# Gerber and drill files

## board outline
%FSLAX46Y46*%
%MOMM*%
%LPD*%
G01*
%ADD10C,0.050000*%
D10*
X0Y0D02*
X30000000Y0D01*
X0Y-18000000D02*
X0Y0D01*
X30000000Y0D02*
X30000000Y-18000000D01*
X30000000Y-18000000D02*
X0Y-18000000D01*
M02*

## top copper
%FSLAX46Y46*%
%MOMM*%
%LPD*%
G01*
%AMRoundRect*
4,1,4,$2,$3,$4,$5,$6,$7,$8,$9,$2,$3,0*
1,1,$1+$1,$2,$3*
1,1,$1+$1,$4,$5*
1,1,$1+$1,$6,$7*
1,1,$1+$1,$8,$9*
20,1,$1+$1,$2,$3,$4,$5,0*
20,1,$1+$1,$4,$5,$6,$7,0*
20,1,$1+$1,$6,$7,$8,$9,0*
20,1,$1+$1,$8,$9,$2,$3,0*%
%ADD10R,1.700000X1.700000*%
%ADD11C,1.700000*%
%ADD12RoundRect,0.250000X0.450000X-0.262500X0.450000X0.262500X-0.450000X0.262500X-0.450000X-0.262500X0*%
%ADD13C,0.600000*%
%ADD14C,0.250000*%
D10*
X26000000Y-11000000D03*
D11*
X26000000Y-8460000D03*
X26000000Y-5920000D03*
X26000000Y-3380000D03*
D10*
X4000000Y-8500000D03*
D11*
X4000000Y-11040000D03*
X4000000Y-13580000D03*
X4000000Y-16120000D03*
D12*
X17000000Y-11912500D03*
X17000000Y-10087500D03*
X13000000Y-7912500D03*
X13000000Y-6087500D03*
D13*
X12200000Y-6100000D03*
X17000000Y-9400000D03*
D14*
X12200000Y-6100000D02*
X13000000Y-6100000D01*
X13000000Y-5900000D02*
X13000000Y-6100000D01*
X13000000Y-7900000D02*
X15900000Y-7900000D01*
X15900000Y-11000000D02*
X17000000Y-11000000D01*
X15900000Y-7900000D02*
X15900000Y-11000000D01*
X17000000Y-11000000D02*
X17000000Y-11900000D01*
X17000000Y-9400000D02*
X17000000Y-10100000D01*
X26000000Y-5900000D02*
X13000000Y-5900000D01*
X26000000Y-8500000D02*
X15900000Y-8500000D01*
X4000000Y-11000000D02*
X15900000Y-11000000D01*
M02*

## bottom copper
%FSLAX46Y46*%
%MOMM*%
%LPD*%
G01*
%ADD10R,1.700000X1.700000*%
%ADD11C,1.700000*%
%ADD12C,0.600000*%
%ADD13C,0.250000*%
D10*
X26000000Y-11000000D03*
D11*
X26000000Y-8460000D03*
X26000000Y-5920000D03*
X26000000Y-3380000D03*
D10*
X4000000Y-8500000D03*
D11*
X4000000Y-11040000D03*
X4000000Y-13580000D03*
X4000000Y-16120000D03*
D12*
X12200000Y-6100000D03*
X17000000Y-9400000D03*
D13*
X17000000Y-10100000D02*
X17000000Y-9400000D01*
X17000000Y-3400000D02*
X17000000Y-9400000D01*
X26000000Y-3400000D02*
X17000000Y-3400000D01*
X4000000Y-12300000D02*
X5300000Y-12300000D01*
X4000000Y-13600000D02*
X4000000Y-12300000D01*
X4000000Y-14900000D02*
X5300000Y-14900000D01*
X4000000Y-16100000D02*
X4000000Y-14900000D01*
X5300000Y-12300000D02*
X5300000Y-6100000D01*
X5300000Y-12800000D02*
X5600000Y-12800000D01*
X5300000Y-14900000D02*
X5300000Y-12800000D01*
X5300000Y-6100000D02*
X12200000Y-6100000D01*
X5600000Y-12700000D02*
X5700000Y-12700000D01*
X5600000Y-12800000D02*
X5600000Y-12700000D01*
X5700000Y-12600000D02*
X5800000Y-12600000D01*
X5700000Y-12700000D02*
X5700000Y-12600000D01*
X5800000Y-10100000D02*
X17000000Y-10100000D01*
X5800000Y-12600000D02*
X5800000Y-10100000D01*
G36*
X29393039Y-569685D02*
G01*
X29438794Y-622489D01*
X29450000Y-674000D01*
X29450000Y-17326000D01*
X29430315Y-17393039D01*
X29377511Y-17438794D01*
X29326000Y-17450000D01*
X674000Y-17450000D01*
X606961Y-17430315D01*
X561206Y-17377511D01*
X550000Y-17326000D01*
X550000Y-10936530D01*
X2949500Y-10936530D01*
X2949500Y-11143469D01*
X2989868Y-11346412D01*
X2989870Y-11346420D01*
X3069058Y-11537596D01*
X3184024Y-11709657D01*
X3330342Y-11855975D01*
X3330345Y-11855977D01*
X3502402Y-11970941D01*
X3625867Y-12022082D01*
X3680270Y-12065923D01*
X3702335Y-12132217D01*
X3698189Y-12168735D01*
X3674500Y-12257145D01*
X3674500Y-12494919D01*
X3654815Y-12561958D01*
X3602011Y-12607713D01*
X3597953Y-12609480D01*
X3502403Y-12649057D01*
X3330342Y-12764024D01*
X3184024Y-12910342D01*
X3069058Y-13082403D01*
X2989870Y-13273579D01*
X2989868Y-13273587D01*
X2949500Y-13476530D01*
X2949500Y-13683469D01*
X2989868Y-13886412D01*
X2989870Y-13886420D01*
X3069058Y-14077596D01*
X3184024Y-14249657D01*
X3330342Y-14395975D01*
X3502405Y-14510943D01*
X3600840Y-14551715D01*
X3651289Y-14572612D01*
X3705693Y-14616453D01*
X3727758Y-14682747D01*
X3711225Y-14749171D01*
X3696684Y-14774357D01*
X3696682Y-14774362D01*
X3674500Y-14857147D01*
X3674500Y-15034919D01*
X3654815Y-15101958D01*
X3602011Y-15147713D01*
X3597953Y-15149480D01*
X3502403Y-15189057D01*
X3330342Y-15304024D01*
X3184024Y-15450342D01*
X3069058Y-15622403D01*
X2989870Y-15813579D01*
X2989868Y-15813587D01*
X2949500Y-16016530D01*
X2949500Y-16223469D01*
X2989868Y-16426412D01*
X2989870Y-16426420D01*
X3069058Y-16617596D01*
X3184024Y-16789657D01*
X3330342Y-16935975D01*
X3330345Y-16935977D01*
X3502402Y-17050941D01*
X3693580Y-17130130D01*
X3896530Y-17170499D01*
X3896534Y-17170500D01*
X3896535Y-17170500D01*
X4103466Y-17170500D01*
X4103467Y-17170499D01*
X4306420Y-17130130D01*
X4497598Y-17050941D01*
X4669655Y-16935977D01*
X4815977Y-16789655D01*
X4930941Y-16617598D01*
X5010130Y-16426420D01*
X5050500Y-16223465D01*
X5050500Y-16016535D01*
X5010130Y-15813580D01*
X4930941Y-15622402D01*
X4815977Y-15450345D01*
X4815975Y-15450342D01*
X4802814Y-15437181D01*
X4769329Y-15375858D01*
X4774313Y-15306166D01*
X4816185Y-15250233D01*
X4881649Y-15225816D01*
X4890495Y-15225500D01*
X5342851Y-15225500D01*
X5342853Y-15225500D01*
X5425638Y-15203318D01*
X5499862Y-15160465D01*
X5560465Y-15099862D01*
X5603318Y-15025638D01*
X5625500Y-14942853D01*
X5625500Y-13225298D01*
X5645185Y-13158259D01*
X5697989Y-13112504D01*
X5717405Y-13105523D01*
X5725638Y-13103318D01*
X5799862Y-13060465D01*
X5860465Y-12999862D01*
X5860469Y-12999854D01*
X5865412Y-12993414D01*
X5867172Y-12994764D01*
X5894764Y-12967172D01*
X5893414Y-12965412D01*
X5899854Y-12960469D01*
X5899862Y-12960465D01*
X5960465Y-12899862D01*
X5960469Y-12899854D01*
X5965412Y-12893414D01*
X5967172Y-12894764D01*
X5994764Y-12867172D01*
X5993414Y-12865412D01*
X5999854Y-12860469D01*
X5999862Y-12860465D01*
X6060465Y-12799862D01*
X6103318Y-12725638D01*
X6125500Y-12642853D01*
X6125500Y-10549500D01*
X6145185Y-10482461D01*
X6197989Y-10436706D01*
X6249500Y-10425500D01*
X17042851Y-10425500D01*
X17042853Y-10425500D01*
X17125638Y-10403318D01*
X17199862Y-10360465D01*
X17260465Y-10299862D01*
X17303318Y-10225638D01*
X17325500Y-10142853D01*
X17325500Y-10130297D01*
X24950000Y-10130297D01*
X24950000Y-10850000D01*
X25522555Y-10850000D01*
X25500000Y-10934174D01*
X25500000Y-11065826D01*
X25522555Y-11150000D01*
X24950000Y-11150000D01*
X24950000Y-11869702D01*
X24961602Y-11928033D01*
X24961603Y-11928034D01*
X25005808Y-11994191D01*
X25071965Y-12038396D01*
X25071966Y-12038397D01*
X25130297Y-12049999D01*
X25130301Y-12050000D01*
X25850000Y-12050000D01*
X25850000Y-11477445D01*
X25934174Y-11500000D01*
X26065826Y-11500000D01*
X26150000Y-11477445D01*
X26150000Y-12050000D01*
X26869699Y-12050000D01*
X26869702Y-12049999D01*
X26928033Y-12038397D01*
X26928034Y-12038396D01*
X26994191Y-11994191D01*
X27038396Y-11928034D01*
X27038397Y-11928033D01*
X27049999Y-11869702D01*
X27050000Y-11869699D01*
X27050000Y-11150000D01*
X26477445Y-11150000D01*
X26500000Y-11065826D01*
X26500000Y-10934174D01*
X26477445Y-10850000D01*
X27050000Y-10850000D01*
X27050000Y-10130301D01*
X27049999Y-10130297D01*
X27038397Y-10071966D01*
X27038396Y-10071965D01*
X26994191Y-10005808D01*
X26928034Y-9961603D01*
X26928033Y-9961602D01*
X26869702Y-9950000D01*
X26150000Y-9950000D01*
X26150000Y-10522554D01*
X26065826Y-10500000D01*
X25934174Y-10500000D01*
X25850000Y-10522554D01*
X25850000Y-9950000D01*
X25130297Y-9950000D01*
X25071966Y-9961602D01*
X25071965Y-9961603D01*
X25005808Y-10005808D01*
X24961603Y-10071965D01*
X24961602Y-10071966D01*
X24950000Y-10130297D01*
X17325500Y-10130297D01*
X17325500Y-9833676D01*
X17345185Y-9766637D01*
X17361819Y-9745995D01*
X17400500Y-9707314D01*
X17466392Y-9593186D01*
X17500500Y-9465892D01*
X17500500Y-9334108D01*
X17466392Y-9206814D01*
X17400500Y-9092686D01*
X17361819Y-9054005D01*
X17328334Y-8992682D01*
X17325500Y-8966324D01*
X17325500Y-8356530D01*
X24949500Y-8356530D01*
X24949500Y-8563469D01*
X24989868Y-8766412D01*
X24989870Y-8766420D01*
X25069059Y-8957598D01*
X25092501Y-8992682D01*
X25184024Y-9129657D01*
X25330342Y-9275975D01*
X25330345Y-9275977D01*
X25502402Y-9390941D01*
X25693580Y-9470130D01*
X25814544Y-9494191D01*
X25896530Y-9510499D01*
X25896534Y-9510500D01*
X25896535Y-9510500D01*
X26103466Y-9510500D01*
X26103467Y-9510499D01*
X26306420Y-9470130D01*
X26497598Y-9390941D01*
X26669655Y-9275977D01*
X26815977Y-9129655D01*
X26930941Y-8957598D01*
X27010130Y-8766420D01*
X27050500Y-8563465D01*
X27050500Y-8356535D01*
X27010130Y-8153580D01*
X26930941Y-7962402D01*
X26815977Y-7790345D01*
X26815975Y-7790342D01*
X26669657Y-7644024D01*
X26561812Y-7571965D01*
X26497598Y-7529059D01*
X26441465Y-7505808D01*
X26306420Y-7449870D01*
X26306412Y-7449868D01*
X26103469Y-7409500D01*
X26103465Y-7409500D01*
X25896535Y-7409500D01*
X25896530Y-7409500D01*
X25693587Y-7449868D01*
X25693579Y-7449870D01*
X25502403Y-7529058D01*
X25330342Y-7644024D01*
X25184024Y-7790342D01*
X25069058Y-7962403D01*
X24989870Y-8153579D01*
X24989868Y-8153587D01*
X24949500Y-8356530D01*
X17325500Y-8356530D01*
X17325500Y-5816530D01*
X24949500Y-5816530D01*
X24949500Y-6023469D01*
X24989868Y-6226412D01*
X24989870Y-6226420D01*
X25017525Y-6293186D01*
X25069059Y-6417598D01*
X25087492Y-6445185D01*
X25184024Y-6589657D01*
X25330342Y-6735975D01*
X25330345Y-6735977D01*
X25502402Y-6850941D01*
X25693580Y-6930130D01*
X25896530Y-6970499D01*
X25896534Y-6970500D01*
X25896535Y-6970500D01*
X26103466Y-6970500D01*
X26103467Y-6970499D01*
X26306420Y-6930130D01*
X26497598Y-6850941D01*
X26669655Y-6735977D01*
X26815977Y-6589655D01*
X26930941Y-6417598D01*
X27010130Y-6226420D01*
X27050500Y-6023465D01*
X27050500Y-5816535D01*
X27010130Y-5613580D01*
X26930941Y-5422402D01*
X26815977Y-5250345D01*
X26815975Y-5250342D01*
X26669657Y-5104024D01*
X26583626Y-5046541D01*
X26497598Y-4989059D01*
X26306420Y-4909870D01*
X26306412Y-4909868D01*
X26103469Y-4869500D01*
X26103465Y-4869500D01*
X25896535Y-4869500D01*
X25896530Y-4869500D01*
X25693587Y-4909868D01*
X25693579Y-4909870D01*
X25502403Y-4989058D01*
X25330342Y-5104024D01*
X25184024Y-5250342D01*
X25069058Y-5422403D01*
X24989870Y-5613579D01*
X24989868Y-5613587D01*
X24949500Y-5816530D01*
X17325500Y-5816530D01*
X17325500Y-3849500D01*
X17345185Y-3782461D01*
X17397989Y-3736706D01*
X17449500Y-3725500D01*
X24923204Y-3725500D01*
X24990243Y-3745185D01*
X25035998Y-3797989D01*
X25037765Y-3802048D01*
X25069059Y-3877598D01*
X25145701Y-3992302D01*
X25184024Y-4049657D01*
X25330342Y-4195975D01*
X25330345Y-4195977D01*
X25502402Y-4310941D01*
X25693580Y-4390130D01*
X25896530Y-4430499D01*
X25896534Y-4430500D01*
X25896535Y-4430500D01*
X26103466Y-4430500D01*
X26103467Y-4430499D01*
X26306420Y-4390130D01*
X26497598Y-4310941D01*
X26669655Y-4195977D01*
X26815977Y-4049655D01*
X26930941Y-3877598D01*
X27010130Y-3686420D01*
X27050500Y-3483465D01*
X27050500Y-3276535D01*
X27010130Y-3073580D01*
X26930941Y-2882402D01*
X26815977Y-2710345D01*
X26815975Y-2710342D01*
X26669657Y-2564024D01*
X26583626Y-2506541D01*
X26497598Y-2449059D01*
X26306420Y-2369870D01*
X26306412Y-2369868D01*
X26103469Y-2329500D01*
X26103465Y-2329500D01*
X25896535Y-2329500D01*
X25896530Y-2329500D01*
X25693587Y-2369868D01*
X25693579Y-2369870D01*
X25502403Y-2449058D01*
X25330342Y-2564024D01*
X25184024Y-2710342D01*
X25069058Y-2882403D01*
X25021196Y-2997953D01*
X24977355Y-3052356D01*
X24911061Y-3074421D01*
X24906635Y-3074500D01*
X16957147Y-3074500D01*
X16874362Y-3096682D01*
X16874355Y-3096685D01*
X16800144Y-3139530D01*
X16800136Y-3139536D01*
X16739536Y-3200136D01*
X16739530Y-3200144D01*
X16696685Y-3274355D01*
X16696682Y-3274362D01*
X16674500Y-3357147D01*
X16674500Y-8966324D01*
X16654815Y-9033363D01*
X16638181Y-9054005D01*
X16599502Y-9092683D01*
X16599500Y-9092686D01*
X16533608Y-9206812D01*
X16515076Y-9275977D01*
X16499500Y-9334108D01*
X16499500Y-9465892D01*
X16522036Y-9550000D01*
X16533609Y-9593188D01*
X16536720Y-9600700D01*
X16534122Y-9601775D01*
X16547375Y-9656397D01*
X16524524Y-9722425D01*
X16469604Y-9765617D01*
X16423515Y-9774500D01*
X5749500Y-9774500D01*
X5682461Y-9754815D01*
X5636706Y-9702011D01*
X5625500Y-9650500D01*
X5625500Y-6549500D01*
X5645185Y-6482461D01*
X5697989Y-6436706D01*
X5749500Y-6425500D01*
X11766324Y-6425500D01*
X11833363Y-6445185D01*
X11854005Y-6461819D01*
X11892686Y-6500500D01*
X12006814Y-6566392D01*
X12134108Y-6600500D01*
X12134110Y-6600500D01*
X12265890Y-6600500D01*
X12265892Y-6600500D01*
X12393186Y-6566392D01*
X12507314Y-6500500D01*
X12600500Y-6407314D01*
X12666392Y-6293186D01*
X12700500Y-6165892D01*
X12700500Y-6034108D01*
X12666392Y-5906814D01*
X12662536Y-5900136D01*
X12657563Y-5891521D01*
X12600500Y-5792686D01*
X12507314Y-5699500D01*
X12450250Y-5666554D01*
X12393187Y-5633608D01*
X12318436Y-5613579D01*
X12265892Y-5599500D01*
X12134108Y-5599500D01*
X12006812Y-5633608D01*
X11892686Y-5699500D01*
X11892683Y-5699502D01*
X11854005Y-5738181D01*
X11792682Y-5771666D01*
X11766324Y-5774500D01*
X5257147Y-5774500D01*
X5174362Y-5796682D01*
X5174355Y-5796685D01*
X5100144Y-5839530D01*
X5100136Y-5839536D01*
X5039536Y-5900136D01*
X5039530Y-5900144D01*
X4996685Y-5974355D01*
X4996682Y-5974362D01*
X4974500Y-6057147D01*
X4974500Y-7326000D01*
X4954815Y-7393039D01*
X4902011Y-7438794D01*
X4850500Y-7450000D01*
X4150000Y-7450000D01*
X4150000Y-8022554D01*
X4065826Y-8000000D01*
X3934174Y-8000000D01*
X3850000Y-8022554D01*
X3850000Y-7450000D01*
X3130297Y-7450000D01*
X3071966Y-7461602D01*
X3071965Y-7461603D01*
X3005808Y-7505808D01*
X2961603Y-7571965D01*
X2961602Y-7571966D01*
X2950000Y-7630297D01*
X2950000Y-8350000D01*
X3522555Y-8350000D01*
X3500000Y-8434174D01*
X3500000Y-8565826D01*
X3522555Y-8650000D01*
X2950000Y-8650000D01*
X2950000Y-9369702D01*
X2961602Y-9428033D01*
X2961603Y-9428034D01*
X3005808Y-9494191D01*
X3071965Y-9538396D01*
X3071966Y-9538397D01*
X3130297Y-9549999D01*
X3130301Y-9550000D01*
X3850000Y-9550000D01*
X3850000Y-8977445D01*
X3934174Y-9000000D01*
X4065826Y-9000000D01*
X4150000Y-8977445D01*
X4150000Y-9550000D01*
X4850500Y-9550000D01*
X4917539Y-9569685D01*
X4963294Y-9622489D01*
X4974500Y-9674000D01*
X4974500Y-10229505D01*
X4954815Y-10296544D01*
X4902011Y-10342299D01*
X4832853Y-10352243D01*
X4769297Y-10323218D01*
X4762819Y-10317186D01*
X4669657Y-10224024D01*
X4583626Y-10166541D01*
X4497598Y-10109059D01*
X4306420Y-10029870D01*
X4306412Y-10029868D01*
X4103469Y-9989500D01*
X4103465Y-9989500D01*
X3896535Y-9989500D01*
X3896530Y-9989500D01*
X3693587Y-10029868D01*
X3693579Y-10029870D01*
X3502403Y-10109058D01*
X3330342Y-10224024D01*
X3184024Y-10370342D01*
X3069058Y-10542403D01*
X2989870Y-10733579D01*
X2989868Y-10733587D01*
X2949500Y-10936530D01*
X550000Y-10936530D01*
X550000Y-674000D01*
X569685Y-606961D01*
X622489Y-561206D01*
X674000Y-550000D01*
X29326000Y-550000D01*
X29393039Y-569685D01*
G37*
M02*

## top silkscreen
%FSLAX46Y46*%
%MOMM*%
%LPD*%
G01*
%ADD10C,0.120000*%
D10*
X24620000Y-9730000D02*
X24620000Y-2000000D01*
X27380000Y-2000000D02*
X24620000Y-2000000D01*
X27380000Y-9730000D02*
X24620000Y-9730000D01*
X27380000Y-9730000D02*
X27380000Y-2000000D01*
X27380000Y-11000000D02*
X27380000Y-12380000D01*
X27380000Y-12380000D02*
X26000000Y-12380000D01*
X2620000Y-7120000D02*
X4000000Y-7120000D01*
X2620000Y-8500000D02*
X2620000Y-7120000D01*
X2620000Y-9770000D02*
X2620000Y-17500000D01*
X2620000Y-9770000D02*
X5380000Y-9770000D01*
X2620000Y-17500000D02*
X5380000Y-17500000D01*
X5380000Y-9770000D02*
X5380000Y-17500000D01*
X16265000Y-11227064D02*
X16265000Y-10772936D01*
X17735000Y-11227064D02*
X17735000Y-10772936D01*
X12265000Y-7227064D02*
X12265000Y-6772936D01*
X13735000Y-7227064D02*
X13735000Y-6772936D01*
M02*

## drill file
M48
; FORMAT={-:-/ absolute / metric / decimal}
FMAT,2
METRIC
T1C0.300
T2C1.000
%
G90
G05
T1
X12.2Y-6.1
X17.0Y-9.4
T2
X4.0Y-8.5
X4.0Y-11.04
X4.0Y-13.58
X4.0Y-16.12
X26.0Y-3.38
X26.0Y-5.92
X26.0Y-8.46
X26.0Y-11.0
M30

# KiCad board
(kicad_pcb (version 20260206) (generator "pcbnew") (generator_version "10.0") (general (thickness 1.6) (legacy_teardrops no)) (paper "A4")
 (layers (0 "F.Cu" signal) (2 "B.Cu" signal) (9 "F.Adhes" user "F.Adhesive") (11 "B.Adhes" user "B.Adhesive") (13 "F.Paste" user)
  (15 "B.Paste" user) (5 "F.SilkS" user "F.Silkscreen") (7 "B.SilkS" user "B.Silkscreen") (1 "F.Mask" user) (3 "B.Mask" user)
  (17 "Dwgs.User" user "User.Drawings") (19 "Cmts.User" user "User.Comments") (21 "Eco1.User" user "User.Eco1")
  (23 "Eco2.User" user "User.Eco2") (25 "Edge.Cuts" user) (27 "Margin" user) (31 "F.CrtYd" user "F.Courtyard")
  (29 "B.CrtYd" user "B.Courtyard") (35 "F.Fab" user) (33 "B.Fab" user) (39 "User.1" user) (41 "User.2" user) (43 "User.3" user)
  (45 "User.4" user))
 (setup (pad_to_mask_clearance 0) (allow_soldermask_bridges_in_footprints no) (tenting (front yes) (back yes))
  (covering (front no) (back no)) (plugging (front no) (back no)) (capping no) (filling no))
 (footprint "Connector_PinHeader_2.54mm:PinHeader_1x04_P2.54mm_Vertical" (layer "F.Cu") (at 26 11 180)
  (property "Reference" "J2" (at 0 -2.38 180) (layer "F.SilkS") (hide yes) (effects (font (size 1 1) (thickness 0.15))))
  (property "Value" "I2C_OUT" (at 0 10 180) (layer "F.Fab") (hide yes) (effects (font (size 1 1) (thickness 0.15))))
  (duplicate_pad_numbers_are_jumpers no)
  (fp_line (start 1.38 1.27) (end 1.38 9) (stroke (width 0.12) (type solid)) (layer "F.SilkS"))
  (fp_line (start -1.38 9) (end 1.38 9) (stroke (width 0.12) (type solid)) (layer "F.SilkS"))
  (fp_line (start -1.38 1.27) (end 1.38 1.27) (stroke (width 0.12) (type solid)) (layer "F.SilkS"))
  (fp_line (start -1.38 1.27) (end -1.38 9) (stroke (width 0.12) (type solid)) (layer "F.SilkS"))
  (fp_line (start -1.38 0) (end -1.38 -1.38) (stroke (width 0.12) (type solid)) (layer "F.SilkS"))
  (fp_line (start -1.38 -1.38) (end 0 -1.38) (stroke (width 0.12) (type solid)) (layer "F.SilkS"))
  (pad "1" thru_hole rect (at 0 0 180) (size 1.7 1.7) (drill 1) (layers "*.Cu" "*.Mask") (remove_unused_layers no) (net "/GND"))
  (pad "2" thru_hole circle (at 0 2.54 180) (size 1.7 1.7) (drill 1) (layers "*.Cu" "*.Mask") (remove_unused_layers no) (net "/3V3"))
  (pad "3" thru_hole circle (at 0 5.08 180) (size 1.7 1.7) (drill 1) (layers "*.Cu" "*.Mask") (remove_unused_layers no) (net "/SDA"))
  (pad "4" thru_hole circle (at 0 7.62 180) (size 1.7 1.7) (drill 1) (layers "*.Cu" "*.Mask") (remove_unused_layers no) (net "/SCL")))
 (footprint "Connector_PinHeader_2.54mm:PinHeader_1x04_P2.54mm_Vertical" (layer "F.Cu") (at 4 8.5)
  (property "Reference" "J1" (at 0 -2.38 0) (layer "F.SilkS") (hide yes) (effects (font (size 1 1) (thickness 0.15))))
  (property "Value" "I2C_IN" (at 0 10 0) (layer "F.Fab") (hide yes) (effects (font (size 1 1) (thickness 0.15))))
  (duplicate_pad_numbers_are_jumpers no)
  (fp_line (start -1.38 -1.38) (end 0 -1.38) (stroke (width 0.12) (type solid)) (layer "F.SilkS"))
  (fp_line (start -1.38 0) (end -1.38 -1.38) (stroke (width 0.12) (type solid)) (layer "F.SilkS"))
  (fp_line (start -1.38 1.27) (end -1.38 9) (stroke (width 0.12) (type solid)) (layer "F.SilkS"))
  (fp_line (start -1.38 1.27) (end 1.38 1.27) (stroke (width 0.12) (type solid)) (layer "F.SilkS"))
  (fp_line (start -1.38 9) (end 1.38 9) (stroke (width 0.12) (type solid)) (layer "F.SilkS"))
  (fp_line (start 1.38 1.27) (end 1.38 9) (stroke (width 0.12) (type solid)) (layer "F.SilkS"))
  (pad "1" thru_hole rect (at 0 0) (size 1.7 1.7) (drill 1) (layers "*.Cu" "*.Mask") (remove_unused_layers no) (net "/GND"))
  (pad "2" thru_hole circle (at 0 2.54) (size 1.7 1.7) (drill 1) (layers "*.Cu" "*.Mask") (remove_unused_layers no) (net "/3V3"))
  (pad "3" thru_hole circle (at 0 5.08) (size 1.7 1.7) (drill 1) (layers "*.Cu" "*.Mask") (remove_unused_layers no) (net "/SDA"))
  (pad "4" thru_hole circle (at 0 7.62) (size 1.7 1.7) (drill 1) (layers "*.Cu" "*.Mask") (remove_unused_layers no) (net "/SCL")))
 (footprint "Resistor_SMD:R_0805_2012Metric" (layer "F.Cu") (at 17 11 90)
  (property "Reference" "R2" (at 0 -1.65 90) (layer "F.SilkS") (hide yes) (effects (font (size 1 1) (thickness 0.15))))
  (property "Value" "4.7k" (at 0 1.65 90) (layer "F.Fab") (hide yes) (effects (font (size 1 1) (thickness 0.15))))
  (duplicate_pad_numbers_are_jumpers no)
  (fp_line (start -0.227064 -0.735) (end 0.227064 -0.735) (stroke (width 0.12) (type solid)) (layer "F.SilkS"))
  (fp_line (start -0.227064 0.735) (end 0.227064 0.735) (stroke (width 0.12) (type solid)) (layer "F.SilkS"))
  (pad "1" smd roundrect (at -0.9125 0 90) (size 1.025 1.4) (layers "F.Cu" "F.Mask" "F.Paste") (roundrect_rratio 0.243902) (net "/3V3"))
  (pad "2" smd roundrect (at 0.9125 0 90) (size 1.025 1.4) (layers "F.Cu" "F.Mask" "F.Paste") (roundrect_rratio 0.243902) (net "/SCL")))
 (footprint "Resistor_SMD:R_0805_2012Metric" (layer "F.Cu") (at 13 7 90)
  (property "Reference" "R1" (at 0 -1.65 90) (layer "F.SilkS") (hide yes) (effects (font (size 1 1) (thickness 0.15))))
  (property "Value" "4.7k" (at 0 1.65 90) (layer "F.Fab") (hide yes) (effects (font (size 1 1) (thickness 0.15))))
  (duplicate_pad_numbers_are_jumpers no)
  (fp_line (start -0.227064 -0.735) (end 0.227064 -0.735) (stroke (width 0.12) (type solid)) (layer "F.SilkS"))
  (fp_line (start -0.227064 0.735) (end 0.227064 0.735) (stroke (width 0.12) (type solid)) (layer "F.SilkS"))
  (pad "1" smd roundrect (at -0.9125 0 90) (size 1.025 1.4) (layers "F.Cu" "F.Mask" "F.Paste") (roundrect_rratio 0.243902) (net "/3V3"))
  (pad "2" smd roundrect (at 0.9125 0 90) (size 1.025 1.4) (layers "F.Cu" "F.Mask" "F.Paste") (roundrect_rratio 0.243902) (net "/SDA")))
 (gr_line (start 0 0) (end 30 0) (stroke (width 0.05) (type default)) (layer "Edge.Cuts"))
 (gr_line (start 0 18) (end 0 0) (stroke (width 0.05) (type default)) (layer "Edge.Cuts"))
 (gr_line (start 30 0) (end 30 18) (stroke (width 0.05) (type default)) (layer "Edge.Cuts"))
 (gr_line (start 30 18) (end 0 18) (stroke (width 0.05) (type default)) (layer "Edge.Cuts"))
 (segment (start 12.2 6.1) (end 13 6.1) (width 0.25) (layer "F.Cu") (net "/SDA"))
 (segment (start 13 5.9) (end 13 6.1) (width 0.25) (layer "F.Cu") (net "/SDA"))
 (segment (start 13 7.9) (end 15.9 7.9) (width 0.25) (layer "F.Cu") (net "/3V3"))
 (segment (start 15.9 11) (end 17 11) (width 0.25) (layer "F.Cu") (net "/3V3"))
 (segment (start 15.9 7.9) (end 15.9 11) (width 0.25) (layer "F.Cu") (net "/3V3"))
 (segment (start 17 10.1) (end 17 9.4) (width 0.25) (layer "B.Cu") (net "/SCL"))
 (segment (start 17 11) (end 17 11.9) (width 0.25) (layer "F.Cu") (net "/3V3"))
 (segment (start 17 3.4) (end 17 9.4) (width 0.25) (layer "B.Cu") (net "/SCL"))
 (segment (start 17 9.4) (end 17 10.1) (width 0.25) (layer "F.Cu") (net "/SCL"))
 (segment (start 26 3.4) (end 17 3.4) (width 0.25) (layer "B.Cu") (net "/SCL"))
 (segment (start 26 5.9) (end 13 5.9) (width 0.25) (layer "F.Cu") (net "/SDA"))
 (segment (start 26 8.5) (end 15.9 8.5) (width 0.25) (layer "F.Cu") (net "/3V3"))
 (segment (start 4 11) (end 15.9 11) (width 0.25) (layer "F.Cu") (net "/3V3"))
 (segment (start 4 12.3) (end 5.3 12.3) (width 0.25) (layer "B.Cu") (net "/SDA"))
 (segment (start 4 13.6) (end 4 12.3) (width 0.25) (layer "B.Cu") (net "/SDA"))
 (segment (start 4 14.9) (end 5.3 14.9) (width 0.25) (layer "B.Cu") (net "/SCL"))
 (segment (start 4 16.1) (end 4 14.9) (width 0.25) (layer "B.Cu") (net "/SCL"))
 (segment (start 5.3 12.3) (end 5.3 6.1) (width 0.25) (layer "B.Cu") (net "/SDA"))
 (segment (start 5.3 12.8) (end 5.6 12.8) (width 0.25) (layer "B.Cu") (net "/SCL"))
 (segment (start 5.3 14.9) (end 5.3 12.8) (width 0.25) (layer "B.Cu") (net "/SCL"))
 (segment (start 5.3 6.1) (end 12.2 6.1) (width 0.25) (layer "B.Cu") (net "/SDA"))
 (segment (start 5.6 12.7) (end 5.7 12.7) (width 0.25) (layer "B.Cu") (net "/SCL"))
 (segment (start 5.6 12.8) (end 5.6 12.7) (width 0.25) (layer "B.Cu") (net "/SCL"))
 (segment (start 5.7 12.6) (end 5.8 12.6) (width 0.25) (layer "B.Cu") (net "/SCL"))
 (segment (start 5.7 12.7) (end 5.7 12.6) (width 0.25) (layer "B.Cu") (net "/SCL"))
 (segment (start 5.8 10.1) (end 17 10.1) (width 0.25) (layer "B.Cu") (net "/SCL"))
 (segment (start 5.8 12.6) (end 5.8 10.1) (width 0.25) (layer "B.Cu") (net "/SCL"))
 (via (at 12.2 6.1) (size 0.6) (drill 0.3) (layers "F.Cu" "B.Cu") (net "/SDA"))
 (via (at 17 9.4) (size 0.6) (drill 0.3) (layers "F.Cu" "B.Cu") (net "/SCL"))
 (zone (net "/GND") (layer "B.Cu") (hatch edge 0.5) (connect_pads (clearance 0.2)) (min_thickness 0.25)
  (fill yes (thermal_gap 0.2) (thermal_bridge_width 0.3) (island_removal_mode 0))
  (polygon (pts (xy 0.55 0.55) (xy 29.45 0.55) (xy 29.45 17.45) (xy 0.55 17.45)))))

